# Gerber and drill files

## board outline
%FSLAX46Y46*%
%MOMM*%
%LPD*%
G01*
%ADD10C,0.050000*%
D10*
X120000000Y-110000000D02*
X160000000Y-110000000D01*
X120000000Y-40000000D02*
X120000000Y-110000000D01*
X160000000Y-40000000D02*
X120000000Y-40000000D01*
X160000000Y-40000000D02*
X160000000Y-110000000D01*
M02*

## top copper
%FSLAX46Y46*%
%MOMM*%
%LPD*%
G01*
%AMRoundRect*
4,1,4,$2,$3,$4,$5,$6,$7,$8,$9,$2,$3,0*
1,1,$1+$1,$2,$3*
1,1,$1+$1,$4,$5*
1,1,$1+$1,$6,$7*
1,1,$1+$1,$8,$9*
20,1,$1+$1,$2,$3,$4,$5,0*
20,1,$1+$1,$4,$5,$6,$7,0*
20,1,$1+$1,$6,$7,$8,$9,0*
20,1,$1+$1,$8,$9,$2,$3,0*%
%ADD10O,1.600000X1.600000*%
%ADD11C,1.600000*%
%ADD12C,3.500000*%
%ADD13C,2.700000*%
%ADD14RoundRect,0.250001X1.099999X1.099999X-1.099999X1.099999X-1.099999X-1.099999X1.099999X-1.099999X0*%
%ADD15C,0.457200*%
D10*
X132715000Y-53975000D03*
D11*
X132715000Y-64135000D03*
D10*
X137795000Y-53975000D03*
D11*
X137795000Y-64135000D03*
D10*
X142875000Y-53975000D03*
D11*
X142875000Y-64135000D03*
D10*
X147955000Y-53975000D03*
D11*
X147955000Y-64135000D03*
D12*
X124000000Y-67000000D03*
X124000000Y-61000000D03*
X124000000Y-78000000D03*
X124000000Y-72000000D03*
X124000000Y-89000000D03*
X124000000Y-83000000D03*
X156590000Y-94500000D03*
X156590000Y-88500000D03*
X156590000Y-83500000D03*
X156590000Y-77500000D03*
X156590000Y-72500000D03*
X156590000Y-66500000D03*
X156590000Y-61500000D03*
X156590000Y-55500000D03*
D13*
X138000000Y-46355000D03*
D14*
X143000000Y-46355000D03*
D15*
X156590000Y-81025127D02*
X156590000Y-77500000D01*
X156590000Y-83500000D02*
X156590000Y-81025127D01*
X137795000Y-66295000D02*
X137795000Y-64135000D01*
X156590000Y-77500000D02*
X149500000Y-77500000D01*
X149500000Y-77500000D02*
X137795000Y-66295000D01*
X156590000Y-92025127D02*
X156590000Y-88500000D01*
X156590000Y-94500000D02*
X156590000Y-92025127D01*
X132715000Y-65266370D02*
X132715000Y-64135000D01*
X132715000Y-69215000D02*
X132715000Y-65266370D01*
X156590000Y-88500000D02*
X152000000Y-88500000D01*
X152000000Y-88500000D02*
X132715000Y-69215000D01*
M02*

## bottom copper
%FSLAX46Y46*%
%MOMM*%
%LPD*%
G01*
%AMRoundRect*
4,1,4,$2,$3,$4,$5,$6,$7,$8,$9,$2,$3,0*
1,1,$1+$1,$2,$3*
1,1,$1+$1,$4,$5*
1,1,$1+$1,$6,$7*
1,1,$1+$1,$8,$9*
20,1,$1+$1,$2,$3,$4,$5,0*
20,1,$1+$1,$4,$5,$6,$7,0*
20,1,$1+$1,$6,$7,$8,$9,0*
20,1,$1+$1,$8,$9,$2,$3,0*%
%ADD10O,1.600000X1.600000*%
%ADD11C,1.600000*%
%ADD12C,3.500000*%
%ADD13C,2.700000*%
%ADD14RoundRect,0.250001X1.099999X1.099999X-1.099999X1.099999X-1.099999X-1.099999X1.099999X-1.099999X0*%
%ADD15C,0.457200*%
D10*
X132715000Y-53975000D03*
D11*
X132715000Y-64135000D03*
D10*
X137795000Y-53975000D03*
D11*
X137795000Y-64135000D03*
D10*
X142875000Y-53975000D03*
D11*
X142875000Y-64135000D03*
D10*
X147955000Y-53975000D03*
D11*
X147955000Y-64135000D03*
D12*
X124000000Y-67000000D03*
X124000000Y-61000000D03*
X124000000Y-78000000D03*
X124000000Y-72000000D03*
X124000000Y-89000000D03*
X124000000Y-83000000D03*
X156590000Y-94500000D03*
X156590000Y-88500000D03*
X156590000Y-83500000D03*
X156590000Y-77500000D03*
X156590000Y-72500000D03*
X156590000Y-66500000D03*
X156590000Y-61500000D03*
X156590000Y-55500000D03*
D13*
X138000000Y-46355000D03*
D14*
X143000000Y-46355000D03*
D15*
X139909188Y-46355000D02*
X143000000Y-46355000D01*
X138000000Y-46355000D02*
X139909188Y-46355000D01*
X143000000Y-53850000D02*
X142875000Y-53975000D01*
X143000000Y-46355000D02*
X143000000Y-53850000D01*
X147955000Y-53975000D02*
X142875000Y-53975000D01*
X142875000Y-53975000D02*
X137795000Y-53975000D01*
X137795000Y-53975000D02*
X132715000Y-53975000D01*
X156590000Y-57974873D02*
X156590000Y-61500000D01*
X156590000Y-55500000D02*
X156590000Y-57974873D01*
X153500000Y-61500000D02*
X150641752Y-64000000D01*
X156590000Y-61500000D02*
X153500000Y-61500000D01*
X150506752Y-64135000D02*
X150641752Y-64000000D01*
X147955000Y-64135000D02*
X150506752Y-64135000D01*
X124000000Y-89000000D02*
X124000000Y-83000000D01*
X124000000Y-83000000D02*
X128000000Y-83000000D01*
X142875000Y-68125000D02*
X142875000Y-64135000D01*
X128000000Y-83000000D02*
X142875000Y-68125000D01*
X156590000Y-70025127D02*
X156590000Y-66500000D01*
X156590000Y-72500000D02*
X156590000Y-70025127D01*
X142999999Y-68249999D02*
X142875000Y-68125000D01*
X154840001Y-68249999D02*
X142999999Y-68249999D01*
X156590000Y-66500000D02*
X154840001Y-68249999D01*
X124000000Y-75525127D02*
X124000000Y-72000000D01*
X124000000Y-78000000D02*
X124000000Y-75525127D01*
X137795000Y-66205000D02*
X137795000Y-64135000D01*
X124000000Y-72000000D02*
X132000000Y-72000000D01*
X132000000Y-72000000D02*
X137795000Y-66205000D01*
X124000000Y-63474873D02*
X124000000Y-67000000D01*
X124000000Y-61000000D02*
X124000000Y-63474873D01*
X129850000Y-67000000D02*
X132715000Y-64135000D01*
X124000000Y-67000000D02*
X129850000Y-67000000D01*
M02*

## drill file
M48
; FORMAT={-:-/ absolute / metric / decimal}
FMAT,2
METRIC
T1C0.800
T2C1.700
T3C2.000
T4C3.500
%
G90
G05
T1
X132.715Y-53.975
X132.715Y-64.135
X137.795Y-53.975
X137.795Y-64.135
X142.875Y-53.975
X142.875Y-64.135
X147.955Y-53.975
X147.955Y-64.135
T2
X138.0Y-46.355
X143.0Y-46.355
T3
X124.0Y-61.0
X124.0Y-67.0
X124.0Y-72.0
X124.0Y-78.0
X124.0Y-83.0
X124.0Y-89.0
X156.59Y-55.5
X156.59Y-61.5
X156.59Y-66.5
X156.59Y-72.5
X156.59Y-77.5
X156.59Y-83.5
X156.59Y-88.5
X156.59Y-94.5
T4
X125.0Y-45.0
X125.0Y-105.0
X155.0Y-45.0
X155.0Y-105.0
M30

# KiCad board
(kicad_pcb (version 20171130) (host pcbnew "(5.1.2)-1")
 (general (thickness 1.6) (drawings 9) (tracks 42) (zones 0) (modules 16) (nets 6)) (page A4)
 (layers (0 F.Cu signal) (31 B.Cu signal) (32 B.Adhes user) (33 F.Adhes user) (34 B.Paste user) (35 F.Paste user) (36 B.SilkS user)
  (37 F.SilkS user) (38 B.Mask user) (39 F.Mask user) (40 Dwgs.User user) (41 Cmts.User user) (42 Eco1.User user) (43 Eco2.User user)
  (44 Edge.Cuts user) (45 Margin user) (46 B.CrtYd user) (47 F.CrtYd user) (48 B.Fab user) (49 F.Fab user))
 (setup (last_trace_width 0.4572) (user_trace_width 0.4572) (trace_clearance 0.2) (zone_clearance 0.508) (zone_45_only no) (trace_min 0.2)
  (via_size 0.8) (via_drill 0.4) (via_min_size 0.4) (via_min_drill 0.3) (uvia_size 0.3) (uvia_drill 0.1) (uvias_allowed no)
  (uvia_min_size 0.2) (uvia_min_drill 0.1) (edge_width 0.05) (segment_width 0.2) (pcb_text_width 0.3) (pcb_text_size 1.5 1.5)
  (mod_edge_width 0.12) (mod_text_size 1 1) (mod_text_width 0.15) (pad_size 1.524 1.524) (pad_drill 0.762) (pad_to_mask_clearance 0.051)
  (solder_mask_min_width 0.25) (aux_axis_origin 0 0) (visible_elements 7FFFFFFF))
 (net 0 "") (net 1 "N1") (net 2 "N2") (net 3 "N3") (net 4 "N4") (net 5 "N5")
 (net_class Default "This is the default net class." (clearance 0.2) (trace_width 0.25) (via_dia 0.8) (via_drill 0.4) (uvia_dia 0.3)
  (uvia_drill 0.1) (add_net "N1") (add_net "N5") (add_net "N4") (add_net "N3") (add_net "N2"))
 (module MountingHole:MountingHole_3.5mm (layer F.Cu) (at 155 105)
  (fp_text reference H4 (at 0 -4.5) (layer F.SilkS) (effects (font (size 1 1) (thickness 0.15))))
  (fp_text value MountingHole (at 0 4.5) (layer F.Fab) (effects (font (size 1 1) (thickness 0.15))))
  (pad 1 np_thru_hole circle (at 0 0) (size 3.5 3.5) (drill 3.5) (layers *.Cu *.Mask)))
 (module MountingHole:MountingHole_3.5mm (layer F.Cu) (at 125 105)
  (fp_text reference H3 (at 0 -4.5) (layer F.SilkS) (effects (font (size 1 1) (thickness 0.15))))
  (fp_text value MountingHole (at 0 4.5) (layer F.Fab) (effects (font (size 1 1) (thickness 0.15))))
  (pad 1 np_thru_hole circle (at 0 0) (size 3.5 3.5) (drill 3.5) (layers *.Cu *.Mask)))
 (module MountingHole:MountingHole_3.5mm (layer F.Cu) (at 155 45)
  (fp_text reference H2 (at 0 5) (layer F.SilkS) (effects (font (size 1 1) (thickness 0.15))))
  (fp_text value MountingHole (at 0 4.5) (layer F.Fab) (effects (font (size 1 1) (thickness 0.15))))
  (pad 1 np_thru_hole circle (at 0 0) (size 3.5 3.5) (drill 3.5) (layers *.Cu *.Mask)))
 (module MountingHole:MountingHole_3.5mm (layer F.Cu) (at 125 45)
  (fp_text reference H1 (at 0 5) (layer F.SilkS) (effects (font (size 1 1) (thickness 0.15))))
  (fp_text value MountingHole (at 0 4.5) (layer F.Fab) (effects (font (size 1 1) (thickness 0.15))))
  (pad 1 np_thru_hole circle (at 0 0) (size 3.5 3.5) (drill 3.5) (layers *.Cu *.Mask)))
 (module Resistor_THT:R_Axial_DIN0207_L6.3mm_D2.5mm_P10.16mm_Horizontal (layer F.Cu) (at 132.715 64.135 90)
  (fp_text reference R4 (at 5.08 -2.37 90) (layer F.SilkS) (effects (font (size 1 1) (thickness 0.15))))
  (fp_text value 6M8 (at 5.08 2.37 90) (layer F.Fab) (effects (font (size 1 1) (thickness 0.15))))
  (pad 2 thru_hole oval (at 10.16 0 90) (size 1.6 1.6) (drill 0.8) (layers *.Cu *.Mask) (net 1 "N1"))
  (pad 1 thru_hole circle (at 0 0 90) (size 1.6 1.6) (drill 0.8) (layers *.Cu *.Mask) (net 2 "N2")))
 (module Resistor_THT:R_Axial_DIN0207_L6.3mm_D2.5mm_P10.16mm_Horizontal (layer F.Cu) (at 137.795 64.135 90)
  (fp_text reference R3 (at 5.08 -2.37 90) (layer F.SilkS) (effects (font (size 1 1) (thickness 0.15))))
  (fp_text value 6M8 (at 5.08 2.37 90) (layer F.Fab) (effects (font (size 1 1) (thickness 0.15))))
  (pad 2 thru_hole oval (at 10.16 0 90) (size 1.6 1.6) (drill 0.8) (layers *.Cu *.Mask) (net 1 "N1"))
  (pad 1 thru_hole circle (at 0 0 90) (size 1.6 1.6) (drill 0.8) (layers *.Cu *.Mask) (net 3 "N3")))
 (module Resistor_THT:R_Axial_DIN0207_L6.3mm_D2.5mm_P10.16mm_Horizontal (layer F.Cu) (at 142.875 64.135 90)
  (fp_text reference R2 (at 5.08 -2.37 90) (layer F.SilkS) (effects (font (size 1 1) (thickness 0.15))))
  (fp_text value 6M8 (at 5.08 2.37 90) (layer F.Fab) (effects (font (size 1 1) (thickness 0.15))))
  (pad 2 thru_hole oval (at 10.16 0 90) (size 1.6 1.6) (drill 0.8) (layers *.Cu *.Mask) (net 1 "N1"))
  (pad 1 thru_hole circle (at 0 0 90) (size 1.6 1.6) (drill 0.8) (layers *.Cu *.Mask) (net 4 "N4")))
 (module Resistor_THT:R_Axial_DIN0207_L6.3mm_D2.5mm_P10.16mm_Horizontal (layer F.Cu) (at 147.955 64.135 90)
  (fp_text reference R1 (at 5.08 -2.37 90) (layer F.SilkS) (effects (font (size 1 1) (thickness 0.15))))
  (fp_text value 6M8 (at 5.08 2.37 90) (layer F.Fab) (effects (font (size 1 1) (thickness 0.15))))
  (pad 2 thru_hole oval (at 10.16 0 90) (size 1.6 1.6) (drill 0.8) (layers *.Cu *.Mask) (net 1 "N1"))
  (pad 1 thru_hole circle (at 0 0 90) (size 1.6 1.6) (drill 0.8) (layers *.Cu *.Mask) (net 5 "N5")))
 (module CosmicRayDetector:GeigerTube (layer F.Cu) (at 116 64 90)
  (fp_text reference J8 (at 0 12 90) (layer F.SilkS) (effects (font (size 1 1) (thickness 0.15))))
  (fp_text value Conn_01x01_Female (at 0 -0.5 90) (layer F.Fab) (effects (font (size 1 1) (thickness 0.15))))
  (pad 1 thru_hole circle (at -3 8 90) (size 3.5 3.5) (drill 2) (layers *.Cu *.Mask) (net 2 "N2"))
  (pad 1 thru_hole circle (at 3 8 90) (size 3.5 3.5) (drill 2) (layers *.Cu *.Mask) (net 2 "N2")))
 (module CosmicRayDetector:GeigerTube (layer F.Cu) (at 116 75 90)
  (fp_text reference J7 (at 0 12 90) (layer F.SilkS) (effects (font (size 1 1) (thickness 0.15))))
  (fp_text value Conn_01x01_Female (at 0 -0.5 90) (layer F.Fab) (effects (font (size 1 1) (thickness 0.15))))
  (pad 1 thru_hole circle (at -3 8 90) (size 3.5 3.5) (drill 2) (layers *.Cu *.Mask) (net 3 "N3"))
  (pad 1 thru_hole circle (at 3 8 90) (size 3.5 3.5) (drill 2) (layers *.Cu *.Mask) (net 3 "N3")))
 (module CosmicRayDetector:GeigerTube (layer F.Cu) (at 116 86 90)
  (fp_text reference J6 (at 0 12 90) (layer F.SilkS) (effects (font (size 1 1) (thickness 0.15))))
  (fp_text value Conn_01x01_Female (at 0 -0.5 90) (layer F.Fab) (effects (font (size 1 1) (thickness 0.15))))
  (pad 1 thru_hole circle (at -3 8 90) (size 3.5 3.5) (drill 2) (layers *.Cu *.Mask) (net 4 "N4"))
  (pad 1 thru_hole circle (at 3 8 90) (size 3.5 3.5) (drill 2) (layers *.Cu *.Mask) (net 4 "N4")))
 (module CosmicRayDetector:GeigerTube (layer F.Cu) (at 148.59 91.5 90)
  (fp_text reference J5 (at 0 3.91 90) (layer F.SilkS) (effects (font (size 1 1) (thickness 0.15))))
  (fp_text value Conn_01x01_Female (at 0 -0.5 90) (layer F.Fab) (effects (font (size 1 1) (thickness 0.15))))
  (pad 1 thru_hole circle (at -3 8 90) (size 3.5 3.5) (drill 2) (layers *.Cu *.Mask) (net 2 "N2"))
  (pad 1 thru_hole circle (at 3 8 90) (size 3.5 3.5) (drill 2) (layers *.Cu *.Mask) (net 2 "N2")))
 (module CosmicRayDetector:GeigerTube (layer F.Cu) (at 148.59 80.5 90)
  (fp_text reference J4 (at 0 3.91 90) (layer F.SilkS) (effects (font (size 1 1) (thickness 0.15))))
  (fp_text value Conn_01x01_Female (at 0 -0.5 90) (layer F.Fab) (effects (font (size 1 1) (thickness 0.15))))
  (pad 1 thru_hole circle (at -3 8 90) (size 3.5 3.5) (drill 2) (layers *.Cu *.Mask) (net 3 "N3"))
  (pad 1 thru_hole circle (at 3 8 90) (size 3.5 3.5) (drill 2) (layers *.Cu *.Mask) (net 3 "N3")))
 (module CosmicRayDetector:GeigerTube (layer F.Cu) (at 148.59 69.5 90)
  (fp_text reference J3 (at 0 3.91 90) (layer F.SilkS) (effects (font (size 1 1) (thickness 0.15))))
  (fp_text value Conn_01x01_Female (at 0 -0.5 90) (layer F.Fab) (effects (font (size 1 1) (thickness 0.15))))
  (pad 1 thru_hole circle (at -3 8 90) (size 3.5 3.5) (drill 2) (layers *.Cu *.Mask) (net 4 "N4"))
  (pad 1 thru_hole circle (at 3 8 90) (size 3.5 3.5) (drill 2) (layers *.Cu *.Mask) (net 4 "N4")))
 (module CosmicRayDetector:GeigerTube (layer F.Cu) (at 148.59 58.5 90)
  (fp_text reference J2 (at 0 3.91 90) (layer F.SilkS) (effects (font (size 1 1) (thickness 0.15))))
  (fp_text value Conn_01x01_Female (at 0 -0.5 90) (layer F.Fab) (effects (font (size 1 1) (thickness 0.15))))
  (pad 1 thru_hole circle (at -3 8 90) (size 3.5 3.5) (drill 2) (layers *.Cu *.Mask) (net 5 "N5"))
  (pad 1 thru_hole circle (at 3 8 90) (size 3.5 3.5) (drill 2) (layers *.Cu *.Mask) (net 5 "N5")))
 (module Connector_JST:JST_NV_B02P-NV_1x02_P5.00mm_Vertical (layer F.Cu) (at 143 46.355 180)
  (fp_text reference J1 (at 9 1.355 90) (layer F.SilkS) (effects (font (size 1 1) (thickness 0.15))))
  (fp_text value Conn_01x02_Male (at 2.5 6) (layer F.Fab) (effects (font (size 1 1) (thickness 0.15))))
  (pad 2 thru_hole circle (at 5 0 180) (size 2.7 2.7) (drill 1.7) (layers *.Cu *.Mask) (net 1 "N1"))
  (pad 1 thru_hole roundrect (at 0 0 180) (size 2.7 2.7) (drill 1.7) (layers *.Cu *.Mask) (roundrect_rratio 0.09259299999999999)
   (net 1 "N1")))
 (gr_line (start 120 110) (end 160 110) (layer Edge.Cuts) (width 0.05))
 (gr_line (start 120 40) (end 120 110) (layer Edge.Cuts) (width 0.05))
 (gr_line (start 160 40) (end 120 40) (layer Edge.Cuts) (width 0.05))
 (gr_line (start 160 40) (end 160 110) (layer Edge.Cuts) (width 0.05))
 (segment (start 139.909188 46.355) (end 143 46.355) (width 0.4572) (layer B.Cu) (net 1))
 (segment (start 138 46.355) (end 139.909188 46.355) (width 0.4572) (layer B.Cu) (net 1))
 (segment (start 143 53.85) (end 142.875 53.975) (width 0.4572) (layer B.Cu) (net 1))
 (segment (start 143 46.355) (end 143 53.85) (width 0.4572) (layer B.Cu) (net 1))
 (segment (start 147.955 53.975) (end 142.875 53.975) (width 0.4572) (layer B.Cu) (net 1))
 (segment (start 142.875 53.975) (end 137.795 53.975) (width 0.4572) (layer B.Cu) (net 1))
 (segment (start 137.795 53.975) (end 132.715 53.975) (width 0.4572) (layer B.Cu) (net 1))
 (segment (start 156.59 57.974873) (end 156.59 61.5) (width 0.4572) (layer B.Cu) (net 5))
 (segment (start 156.59 55.5) (end 156.59 57.974873) (width 0.4572) (layer B.Cu) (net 5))
 (segment (start 153.5 61.5) (end 150.641752 64) (width 0.4572) (layer B.Cu) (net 5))
 (segment (start 156.59 61.5) (end 153.5 61.5) (width 0.4572) (layer B.Cu) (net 5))
 (segment (start 150.506752 64.135) (end 150.641752 64) (width 0.4572) (layer B.Cu) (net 5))
 (segment (start 147.955 64.135) (end 150.506752 64.135) (width 0.4572) (layer B.Cu) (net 5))
 (segment (start 124 89) (end 124 83) (width 0.4572) (layer B.Cu) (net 4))
 (segment (start 124 83) (end 128 83) (width 0.4572) (layer B.Cu) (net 4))
 (segment (start 142.875 68.125) (end 142.875 64.135) (width 0.4572) (layer B.Cu) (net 4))
 (segment (start 128 83) (end 142.875 68.125) (width 0.4572) (layer B.Cu) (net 4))
 (segment (start 156.59 70.025127) (end 156.59 66.5) (width 0.4572) (layer B.Cu) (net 4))
 (segment (start 156.59 72.5) (end 156.59 70.025127) (width 0.4572) (layer B.Cu) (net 4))
 (segment (start 142.999999 68.249999) (end 142.875 68.125) (width 0.4572) (layer B.Cu) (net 4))
 (segment (start 154.840001 68.249999) (end 142.999999 68.249999) (width 0.4572) (layer B.Cu) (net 4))
 (segment (start 156.59 66.5) (end 154.840001 68.249999) (width 0.4572) (layer B.Cu) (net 4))
 (segment (start 124 75.525127) (end 124 72) (width 0.4572) (layer B.Cu) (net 3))
 (segment (start 124 78) (end 124 75.525127) (width 0.4572) (layer B.Cu) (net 3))
 (segment (start 137.795 66.205) (end 137.795 64.135) (width 0.4572) (layer B.Cu) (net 3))
 (segment (start 124 72) (end 132 72) (width 0.4572) (layer B.Cu) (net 3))
 (segment (start 132 72) (end 137.795 66.205) (width 0.4572) (layer B.Cu) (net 3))
 (segment (start 156.59 81.025127) (end 156.59 77.5) (width 0.4572) (layer F.Cu) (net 3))
 (segment (start 156.59 83.5) (end 156.59 81.025127) (width 0.4572) (layer F.Cu) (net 3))
 (segment (start 137.795 66.295) (end 137.795 64.135) (width 0.4572) (layer F.Cu) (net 3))
 (segment (start 156.59 77.5) (end 149.5 77.5) (width 0.4572) (layer F.Cu) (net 3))
 (segment (start 149.5 77.5) (end 137.795 66.295) (width 0.4572) (layer F.Cu) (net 3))
 (segment (start 124 63.474873) (end 124 67) (width 0.4572) (layer B.Cu) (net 2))
 (segment (start 124 61) (end 124 63.474873) (width 0.4572) (layer B.Cu) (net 2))
 (segment (start 129.85 67) (end 132.715 64.135) (width 0.4572) (layer B.Cu) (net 2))
 (segment (start 124 67) (end 129.85 67) (width 0.4572) (layer B.Cu) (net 2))
 (segment (start 156.59 92.025127) (end 156.59 88.5) (width 0.4572) (layer F.Cu) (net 2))
 (segment (start 156.59 94.5) (end 156.59 92.025127) (width 0.4572) (layer F.Cu) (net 2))
 (segment (start 132.715 65.26637) (end 132.715 64.135) (width 0.4572) (layer F.Cu) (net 2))
 (segment (start 132.715 69.215) (end 132.715 65.26637) (width 0.4572) (layer F.Cu) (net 2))
 (segment (start 156.59 88.5) (end 152 88.5) (width 0.4572) (layer F.Cu) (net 2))
 (segment (start 152 88.5) (end 132.715 69.215) (width 0.4572) (layer F.Cu) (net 2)))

